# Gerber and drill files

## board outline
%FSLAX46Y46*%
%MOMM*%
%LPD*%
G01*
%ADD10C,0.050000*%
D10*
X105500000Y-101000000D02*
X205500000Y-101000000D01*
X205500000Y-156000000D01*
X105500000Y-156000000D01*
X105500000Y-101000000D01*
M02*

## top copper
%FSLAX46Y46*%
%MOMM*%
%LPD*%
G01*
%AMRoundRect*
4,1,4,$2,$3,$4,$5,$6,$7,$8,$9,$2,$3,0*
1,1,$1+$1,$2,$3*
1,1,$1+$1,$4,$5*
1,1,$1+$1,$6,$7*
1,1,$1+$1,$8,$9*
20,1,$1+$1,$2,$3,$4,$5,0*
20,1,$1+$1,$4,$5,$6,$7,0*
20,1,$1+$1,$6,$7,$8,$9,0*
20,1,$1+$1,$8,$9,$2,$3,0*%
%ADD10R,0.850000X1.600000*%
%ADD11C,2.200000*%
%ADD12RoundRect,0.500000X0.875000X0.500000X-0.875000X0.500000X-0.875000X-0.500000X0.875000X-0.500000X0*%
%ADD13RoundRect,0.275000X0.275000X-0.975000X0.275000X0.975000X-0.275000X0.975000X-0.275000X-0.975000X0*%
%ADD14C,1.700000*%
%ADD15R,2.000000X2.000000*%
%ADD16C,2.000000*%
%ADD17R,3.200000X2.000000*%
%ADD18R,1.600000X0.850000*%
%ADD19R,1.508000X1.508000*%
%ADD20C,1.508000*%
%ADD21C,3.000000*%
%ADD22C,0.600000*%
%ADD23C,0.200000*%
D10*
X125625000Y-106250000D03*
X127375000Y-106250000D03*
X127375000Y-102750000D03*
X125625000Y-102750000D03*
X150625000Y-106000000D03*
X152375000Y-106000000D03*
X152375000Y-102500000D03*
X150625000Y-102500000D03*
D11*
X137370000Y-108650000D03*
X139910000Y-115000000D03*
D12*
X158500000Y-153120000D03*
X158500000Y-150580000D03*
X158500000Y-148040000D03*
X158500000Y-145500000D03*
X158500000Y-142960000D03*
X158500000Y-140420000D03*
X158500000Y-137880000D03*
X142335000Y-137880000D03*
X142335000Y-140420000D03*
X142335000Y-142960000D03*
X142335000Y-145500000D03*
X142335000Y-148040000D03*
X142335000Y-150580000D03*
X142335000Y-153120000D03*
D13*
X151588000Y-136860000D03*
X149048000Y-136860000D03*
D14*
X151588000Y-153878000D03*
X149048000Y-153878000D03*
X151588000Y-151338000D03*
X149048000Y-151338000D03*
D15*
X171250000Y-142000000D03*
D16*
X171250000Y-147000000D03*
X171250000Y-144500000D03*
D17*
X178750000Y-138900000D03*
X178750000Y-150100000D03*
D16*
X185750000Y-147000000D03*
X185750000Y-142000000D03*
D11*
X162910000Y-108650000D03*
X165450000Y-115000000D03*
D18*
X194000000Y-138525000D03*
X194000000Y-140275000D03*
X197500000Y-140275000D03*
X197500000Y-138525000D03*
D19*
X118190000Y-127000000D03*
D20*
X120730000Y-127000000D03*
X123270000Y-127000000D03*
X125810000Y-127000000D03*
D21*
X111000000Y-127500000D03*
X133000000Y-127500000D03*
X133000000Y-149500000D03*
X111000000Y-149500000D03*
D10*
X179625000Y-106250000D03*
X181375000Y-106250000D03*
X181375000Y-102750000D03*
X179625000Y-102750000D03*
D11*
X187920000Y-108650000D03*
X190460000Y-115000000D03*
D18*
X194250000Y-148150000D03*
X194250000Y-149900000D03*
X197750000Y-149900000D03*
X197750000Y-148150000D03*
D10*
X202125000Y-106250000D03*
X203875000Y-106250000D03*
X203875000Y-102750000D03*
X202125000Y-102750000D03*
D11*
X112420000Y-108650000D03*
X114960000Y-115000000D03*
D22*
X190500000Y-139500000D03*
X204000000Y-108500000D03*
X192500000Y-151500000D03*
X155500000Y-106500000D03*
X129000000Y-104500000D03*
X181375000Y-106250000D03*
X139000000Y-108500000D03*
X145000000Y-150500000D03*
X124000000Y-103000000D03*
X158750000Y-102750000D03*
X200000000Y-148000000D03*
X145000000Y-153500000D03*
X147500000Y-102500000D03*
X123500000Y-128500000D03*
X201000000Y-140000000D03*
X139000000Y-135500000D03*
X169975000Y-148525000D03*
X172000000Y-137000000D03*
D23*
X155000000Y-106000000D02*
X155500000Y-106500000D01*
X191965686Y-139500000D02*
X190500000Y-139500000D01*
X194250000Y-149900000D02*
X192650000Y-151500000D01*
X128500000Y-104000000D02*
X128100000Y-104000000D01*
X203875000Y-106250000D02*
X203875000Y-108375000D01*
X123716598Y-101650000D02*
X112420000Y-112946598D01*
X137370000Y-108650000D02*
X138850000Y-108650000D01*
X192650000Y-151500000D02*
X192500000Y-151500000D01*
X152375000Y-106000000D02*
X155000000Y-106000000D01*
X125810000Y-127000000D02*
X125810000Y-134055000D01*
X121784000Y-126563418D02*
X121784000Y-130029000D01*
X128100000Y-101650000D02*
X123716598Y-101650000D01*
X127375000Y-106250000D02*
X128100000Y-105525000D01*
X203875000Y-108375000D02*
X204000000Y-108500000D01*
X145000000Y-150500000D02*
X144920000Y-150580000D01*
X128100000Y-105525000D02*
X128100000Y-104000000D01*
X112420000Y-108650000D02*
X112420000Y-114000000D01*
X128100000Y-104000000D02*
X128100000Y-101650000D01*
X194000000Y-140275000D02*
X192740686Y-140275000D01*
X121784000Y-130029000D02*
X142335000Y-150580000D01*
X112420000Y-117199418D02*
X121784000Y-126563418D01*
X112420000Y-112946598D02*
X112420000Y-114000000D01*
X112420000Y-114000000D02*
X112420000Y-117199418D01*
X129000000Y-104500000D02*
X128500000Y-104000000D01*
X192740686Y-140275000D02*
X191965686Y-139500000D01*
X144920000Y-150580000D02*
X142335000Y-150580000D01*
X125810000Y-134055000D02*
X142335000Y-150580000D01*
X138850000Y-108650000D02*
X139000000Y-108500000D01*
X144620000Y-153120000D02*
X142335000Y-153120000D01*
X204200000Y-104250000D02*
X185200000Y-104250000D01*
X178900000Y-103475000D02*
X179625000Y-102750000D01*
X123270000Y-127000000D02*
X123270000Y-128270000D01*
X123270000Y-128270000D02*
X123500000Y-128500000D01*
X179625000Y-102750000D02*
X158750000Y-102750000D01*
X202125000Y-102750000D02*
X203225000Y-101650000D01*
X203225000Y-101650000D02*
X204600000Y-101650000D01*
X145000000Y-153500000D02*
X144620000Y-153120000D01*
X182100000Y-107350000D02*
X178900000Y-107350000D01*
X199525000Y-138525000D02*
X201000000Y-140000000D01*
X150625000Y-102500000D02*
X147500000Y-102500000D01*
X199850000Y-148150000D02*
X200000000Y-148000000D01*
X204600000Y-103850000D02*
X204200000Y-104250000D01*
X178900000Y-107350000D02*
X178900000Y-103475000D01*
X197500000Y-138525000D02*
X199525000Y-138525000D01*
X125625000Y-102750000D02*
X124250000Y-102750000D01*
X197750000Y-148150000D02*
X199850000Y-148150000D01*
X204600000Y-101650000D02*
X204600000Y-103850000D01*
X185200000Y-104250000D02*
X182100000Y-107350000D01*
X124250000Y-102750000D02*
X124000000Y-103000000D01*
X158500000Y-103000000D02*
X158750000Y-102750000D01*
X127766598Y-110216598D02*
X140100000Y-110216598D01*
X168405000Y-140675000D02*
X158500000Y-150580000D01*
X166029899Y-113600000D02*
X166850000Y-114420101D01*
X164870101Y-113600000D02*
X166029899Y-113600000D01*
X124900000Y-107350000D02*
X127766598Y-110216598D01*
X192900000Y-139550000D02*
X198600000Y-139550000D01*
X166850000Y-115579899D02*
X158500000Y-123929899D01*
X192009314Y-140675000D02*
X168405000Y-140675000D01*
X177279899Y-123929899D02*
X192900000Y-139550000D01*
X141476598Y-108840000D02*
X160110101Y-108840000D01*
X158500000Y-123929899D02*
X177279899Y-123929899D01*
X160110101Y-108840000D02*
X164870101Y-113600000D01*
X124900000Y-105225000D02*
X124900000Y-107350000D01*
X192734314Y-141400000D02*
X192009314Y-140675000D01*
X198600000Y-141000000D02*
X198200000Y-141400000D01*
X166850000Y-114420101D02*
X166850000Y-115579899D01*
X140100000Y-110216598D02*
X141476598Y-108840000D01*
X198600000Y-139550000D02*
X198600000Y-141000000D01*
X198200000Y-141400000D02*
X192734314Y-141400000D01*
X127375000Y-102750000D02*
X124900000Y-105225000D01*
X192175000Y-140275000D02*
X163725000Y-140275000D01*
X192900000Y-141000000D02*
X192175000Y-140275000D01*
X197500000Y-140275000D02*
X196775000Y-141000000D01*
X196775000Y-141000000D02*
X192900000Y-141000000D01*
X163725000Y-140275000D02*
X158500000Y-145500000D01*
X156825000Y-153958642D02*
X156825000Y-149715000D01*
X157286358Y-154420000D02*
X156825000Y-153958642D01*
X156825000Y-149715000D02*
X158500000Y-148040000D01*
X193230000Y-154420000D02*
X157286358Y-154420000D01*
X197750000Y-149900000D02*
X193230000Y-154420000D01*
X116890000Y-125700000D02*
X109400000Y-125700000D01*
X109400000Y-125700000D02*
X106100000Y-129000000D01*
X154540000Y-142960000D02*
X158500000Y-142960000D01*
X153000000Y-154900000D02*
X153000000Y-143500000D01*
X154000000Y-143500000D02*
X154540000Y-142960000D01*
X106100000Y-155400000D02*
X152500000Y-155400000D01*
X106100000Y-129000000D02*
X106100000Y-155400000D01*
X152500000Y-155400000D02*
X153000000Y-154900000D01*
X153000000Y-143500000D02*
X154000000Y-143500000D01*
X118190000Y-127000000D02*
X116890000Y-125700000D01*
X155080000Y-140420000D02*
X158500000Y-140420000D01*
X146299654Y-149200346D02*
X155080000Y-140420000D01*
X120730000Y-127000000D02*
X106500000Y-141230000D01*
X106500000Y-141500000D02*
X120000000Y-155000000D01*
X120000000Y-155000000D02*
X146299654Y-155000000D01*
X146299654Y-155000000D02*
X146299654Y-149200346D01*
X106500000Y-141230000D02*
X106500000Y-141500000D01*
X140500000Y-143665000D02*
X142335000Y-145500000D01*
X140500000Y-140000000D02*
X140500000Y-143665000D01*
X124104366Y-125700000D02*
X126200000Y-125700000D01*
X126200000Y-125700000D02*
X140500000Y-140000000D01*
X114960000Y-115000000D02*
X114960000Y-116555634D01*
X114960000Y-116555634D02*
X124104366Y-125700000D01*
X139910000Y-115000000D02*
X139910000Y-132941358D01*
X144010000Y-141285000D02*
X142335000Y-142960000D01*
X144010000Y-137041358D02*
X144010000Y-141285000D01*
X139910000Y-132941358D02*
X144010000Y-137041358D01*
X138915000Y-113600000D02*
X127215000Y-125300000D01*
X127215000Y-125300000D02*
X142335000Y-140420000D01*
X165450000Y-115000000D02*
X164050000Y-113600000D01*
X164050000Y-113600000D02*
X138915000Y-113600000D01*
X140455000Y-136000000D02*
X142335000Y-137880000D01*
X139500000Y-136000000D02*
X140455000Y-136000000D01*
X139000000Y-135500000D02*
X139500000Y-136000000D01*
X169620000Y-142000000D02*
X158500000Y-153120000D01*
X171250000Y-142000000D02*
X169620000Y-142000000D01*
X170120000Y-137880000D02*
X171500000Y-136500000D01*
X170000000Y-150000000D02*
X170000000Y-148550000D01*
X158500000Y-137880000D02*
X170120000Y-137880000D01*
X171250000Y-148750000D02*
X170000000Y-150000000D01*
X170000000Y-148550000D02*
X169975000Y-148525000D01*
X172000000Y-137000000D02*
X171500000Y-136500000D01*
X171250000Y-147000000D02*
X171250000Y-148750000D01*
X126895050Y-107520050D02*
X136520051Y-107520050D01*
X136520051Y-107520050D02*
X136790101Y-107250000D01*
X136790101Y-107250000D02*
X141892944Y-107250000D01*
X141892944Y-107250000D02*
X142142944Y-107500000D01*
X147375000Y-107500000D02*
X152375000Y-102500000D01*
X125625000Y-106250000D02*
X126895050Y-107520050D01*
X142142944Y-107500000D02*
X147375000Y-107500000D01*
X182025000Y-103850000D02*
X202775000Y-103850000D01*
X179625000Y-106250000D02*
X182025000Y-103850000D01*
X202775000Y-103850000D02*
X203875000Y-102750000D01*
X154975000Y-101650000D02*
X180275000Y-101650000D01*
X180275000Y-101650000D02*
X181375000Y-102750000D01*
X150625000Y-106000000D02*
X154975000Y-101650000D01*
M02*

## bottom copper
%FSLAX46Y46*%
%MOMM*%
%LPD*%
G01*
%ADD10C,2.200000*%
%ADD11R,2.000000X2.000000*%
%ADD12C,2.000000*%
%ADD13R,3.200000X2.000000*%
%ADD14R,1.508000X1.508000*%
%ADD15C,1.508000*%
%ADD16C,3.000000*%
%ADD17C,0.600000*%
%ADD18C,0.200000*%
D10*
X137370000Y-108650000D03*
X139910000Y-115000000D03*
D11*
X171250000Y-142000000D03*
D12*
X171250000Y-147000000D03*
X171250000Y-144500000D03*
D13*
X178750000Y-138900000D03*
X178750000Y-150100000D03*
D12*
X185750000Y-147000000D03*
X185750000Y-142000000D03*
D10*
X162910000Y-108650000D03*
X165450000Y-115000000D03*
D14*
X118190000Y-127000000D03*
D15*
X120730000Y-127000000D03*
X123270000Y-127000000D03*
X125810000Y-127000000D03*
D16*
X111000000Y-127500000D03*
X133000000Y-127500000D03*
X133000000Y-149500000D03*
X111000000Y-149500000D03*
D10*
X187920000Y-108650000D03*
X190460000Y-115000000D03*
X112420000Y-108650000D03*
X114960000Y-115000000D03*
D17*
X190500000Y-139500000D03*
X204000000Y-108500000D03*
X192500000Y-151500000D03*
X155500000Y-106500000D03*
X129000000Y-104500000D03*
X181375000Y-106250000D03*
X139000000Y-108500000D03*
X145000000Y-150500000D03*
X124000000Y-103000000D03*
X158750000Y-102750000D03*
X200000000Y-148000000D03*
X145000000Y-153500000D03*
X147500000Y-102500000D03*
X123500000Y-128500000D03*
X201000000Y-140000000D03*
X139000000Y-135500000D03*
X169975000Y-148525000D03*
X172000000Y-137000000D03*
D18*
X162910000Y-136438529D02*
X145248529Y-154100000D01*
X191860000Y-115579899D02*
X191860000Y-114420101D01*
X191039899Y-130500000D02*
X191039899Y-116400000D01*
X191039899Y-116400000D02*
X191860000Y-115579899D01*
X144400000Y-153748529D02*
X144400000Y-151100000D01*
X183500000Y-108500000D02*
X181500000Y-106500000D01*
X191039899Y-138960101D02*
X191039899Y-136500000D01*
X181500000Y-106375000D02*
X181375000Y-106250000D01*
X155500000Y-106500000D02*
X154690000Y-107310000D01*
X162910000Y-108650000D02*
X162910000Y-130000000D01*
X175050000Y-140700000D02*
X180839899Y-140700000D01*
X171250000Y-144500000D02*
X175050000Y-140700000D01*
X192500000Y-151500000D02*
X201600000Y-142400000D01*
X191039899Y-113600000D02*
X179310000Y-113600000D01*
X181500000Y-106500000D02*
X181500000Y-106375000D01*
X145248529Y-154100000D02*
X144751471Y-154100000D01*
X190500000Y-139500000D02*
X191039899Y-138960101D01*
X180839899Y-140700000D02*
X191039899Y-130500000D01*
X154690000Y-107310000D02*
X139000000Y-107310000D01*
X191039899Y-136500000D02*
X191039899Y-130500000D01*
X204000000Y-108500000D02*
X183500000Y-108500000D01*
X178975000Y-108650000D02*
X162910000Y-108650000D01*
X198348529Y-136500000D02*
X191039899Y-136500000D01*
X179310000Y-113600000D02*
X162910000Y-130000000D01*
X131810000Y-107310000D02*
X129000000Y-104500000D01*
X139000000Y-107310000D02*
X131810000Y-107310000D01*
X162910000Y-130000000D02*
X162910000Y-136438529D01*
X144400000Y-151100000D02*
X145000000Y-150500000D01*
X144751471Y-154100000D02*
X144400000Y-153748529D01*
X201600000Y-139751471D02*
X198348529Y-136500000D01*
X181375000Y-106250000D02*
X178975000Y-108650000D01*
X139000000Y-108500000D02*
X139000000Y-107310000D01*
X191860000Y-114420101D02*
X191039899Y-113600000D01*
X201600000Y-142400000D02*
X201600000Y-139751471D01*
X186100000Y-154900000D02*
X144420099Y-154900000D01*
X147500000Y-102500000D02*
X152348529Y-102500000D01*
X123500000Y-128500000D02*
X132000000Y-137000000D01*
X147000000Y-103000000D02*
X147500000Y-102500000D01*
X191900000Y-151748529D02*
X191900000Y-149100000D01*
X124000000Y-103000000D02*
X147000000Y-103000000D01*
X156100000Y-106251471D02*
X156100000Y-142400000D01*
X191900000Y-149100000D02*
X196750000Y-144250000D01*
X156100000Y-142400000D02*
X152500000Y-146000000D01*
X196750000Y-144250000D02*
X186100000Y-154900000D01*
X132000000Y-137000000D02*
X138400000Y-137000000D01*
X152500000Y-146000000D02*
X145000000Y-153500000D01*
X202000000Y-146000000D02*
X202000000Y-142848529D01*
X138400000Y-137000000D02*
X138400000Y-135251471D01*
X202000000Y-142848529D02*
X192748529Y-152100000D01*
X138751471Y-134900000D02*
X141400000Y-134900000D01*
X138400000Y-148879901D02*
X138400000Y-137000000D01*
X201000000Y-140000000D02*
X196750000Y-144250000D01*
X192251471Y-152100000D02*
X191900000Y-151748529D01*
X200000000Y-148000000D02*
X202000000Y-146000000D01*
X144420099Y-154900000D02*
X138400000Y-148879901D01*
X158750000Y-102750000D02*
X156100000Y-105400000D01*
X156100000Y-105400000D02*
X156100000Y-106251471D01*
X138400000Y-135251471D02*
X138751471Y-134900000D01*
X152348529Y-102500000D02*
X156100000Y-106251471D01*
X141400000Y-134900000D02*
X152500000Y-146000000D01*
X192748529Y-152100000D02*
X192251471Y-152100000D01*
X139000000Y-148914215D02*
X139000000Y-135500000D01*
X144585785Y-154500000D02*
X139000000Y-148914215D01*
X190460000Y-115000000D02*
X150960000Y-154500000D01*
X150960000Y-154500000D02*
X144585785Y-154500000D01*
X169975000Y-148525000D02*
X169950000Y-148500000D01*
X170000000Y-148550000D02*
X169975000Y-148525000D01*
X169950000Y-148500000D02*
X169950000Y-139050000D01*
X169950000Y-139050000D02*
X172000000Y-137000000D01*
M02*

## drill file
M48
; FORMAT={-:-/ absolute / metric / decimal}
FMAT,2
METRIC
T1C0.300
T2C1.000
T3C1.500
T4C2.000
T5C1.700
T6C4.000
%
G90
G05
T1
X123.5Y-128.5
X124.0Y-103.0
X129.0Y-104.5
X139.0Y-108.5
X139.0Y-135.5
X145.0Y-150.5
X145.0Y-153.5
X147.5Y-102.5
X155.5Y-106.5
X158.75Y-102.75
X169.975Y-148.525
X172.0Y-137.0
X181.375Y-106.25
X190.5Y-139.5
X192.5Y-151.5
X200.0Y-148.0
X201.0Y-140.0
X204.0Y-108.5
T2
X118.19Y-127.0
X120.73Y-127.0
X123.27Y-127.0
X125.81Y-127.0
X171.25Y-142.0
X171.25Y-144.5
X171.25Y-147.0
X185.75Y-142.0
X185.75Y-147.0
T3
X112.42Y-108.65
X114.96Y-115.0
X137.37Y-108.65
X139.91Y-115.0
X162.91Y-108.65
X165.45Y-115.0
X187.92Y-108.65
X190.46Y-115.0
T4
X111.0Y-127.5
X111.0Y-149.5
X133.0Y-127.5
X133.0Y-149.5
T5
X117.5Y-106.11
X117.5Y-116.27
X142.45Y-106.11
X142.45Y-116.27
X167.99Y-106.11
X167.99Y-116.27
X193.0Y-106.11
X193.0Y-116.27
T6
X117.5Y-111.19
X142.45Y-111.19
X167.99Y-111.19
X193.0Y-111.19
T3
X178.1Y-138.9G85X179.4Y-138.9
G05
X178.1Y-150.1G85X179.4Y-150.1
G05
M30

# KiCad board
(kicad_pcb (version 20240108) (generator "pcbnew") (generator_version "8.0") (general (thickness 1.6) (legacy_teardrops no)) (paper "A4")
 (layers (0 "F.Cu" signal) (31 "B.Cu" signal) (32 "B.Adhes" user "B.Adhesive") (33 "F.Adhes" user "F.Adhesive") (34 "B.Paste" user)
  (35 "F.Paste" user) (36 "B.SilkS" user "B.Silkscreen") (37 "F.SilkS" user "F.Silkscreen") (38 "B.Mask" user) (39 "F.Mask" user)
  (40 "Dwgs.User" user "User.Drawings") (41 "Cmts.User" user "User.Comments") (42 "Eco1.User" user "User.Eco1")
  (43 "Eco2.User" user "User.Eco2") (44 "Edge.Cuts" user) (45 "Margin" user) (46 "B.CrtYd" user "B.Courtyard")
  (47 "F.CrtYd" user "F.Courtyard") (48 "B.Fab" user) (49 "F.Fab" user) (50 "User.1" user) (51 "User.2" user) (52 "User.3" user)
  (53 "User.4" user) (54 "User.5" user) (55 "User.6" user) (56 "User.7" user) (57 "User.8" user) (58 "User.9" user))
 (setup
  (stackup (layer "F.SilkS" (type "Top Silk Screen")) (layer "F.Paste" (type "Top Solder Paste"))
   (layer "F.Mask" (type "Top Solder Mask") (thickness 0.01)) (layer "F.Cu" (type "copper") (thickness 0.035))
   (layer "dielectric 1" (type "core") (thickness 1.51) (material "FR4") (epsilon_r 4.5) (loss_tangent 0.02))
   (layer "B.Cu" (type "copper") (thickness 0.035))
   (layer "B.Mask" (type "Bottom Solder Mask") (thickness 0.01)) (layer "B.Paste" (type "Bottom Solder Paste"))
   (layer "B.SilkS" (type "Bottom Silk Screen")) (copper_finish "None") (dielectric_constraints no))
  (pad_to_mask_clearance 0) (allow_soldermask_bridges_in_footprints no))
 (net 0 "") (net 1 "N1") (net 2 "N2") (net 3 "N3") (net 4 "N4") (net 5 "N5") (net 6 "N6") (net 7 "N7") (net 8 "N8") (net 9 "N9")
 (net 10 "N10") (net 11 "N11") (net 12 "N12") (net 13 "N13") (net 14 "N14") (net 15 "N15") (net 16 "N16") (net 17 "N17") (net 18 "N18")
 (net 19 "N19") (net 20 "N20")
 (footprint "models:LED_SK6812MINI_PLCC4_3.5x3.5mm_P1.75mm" (layer "F.Cu") (at 126.5 104.5 90)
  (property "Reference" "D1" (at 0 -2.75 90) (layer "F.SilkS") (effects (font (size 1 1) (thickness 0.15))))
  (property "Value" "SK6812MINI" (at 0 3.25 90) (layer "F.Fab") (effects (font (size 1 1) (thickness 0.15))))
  (pad "1" smd rect (at -1.75 -0.875 90) (size 1.6 0.85) (layers "F.Cu" "F.Paste" "F.Mask") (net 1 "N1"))
  (pad "2" smd rect (at -1.75 0.875 90) (size 1.6 0.85) (layers "F.Cu" "F.Paste" "F.Mask") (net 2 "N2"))
  (pad "3" smd rect (at 1.75 0.875 90) (size 1.6 0.85) (layers "F.Cu" "F.Paste" "F.Mask") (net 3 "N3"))
  (pad "4" smd rect (at 1.75 -0.875 90) (size 1.6 0.85) (layers "F.Cu" "F.Paste" "F.Mask") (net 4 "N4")))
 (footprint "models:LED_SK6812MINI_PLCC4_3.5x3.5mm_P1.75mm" (layer "F.Cu") (at 151.5 104.25 90)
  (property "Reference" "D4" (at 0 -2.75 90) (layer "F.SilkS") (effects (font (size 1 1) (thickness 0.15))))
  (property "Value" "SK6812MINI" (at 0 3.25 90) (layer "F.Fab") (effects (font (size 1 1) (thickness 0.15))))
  (pad "1" smd rect (at -1.75 -0.875 90) (size 1.6 0.85) (layers "F.Cu" "F.Paste" "F.Mask") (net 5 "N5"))
  (pad "2" smd rect (at -1.75 0.875 90) (size 1.6 0.85) (layers "F.Cu" "F.Paste" "F.Mask") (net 2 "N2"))
  (pad "3" smd rect (at 1.75 0.875 90) (size 1.6 0.85) (layers "F.Cu" "F.Paste" "F.Mask") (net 1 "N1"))
  (pad "4" smd rect (at 1.75 -0.875 90) (size 1.6 0.85) (layers "F.Cu" "F.Paste" "F.Mask") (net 4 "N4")))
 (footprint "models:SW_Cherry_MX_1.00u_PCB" (layer "F.Cu") (at 137.37 108.65 90)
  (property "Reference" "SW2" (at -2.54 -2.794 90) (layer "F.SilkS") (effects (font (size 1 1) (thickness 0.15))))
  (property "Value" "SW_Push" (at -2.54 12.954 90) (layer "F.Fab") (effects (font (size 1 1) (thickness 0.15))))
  (pad "" np_thru_hole circle (at -7.62 5.08 90) (size 1.7 1.7) (drill 1.7) (layers "*.Cu" "*.Mask"))
  (pad "" np_thru_hole circle (at -2.54 5.08 90) (size 4 4) (drill 4) (layers "*.Cu" "*.Mask"))
  (pad "" np_thru_hole circle (at 2.54 5.08 90) (size 1.7 1.7) (drill 1.7) (layers "*.Cu" "*.Mask"))
  (pad "1" thru_hole circle (at 0 0 90) (size 2.2 2.2) (drill 1.5) (layers "*.Cu" "*.Mask") (remove_unused_layers no) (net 2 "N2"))
  (pad "2" thru_hole circle (at -6.35 2.54 90) (size 2.2 2.2) (drill 1.5) (layers "*.Cu" "*.Mask") (remove_unused_layers no) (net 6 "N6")))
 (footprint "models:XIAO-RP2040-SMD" (layer "F.Cu") (at 150.5 145.5 180)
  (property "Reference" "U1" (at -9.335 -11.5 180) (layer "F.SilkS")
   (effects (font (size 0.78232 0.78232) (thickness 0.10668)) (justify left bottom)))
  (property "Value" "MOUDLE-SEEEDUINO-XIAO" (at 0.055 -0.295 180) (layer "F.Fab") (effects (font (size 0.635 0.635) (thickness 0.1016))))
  (pad "1" smd roundrect (at -8 -7.62 180) (size 2.75 2) (layers "F.Cu" "F.Paste" "F.Mask") (roundrect_rratio 0.25) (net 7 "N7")
   (solder_mask_margin 0.0508) (thermal_bridge_angle 45))
  (pad "2" smd roundrect (at -8 -5.08 180) (size 2.75 2) (layers "F.Cu" "F.Paste" "F.Mask") (roundrect_rratio 0.25) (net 3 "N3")
   (solder_mask_margin 0.0508) (thermal_bridge_angle 45))
  (pad "3" smd roundrect (at -8 -2.54 180) (size 2.75 2) (layers "F.Cu" "F.Paste" "F.Mask") (roundrect_rratio 0.25) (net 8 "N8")
   (solder_mask_margin 0.0508) (thermal_bridge_angle 45))
  (pad "4" smd roundrect (at -8 0 180) (size 2.75 2) (layers "F.Cu" "F.Paste" "F.Mask") (roundrect_rratio 0.25) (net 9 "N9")
   (solder_mask_margin 0.0508) (thermal_bridge_angle 45))
  (pad "5" smd roundrect (at -8 2.54 180) (size 2.75 2) (layers "F.Cu" "F.Paste" "F.Mask") (roundrect_rratio 0.25) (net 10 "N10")
   (solder_mask_margin 0.0508) (thermal_bridge_angle 45))
  (pad "6" smd roundrect (at -8 5.08 180) (size 2.75 2) (layers "F.Cu" "F.Paste" "F.Mask") (roundrect_rratio 0.25) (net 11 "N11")
   (solder_mask_margin 0.0508) (thermal_bridge_angle 45))
  (pad "7" smd roundrect (at -8 7.62 180) (size 2.75 2) (layers "F.Cu" "F.Paste" "F.Mask") (roundrect_rratio 0.25) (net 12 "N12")
   (solder_mask_margin 0.0508) (thermal_bridge_angle 45))
  (pad "8" smd roundrect (at 8.165 7.62 180) (size 2.75 2) (layers "F.Cu" "F.Paste" "F.Mask") (roundrect_rratio 0.25) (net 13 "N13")
   (solder_mask_margin 0.0508) (thermal_bridge_angle 45))
  (pad "9" smd roundrect (at 8.165 5.08 180) (size 2.75 2) (layers "F.Cu" "F.Paste" "F.Mask") (roundrect_rratio 0.25) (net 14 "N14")
   (solder_mask_margin 0.0508) (thermal_bridge_angle 45))
  (pad "10" smd roundrect (at 8.165 2.54 180) (size 2.75 2) (layers "F.Cu" "F.Paste" "F.Mask") (roundrect_rratio 0.25) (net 6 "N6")
   (solder_mask_margin 0.0508) (thermal_bridge_angle 45))
  (pad "11" smd roundrect (at 8.165 0 180) (size 2.75 2) (layers "F.Cu" "F.Paste" "F.Mask") (roundrect_rratio 0.25) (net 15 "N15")
   (solder_mask_margin 0.0508) (thermal_bridge_angle 45))
  (pad "12" smd roundrect (at 8.165 -2.54 180) (size 2.75 2) (layers "F.Cu" "F.Paste" "F.Mask") (roundrect_rratio 0.25) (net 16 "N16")
   (solder_mask_margin 0.0508) (thermal_bridge_angle 45))
  (pad "13" smd roundrect (at 8.165 -5.08 180) (size 2.75 2) (layers "F.Cu" "F.Paste" "F.Mask") (roundrect_rratio 0.25) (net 2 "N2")
   (solder_mask_margin 0.0508) (thermal_bridge_angle 45))
  (pad "14" smd roundrect (at 8.165 -7.62 180) (size 2.75 2) (layers "F.Cu" "F.Paste" "F.Mask") (roundrect_rratio 0.25) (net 4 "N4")
   (solder_mask_margin 0.0508) (thermal_bridge_angle 45))
  (pad "15" smd roundrect (at -1.088 8.64 90) (size 2.5 1.1) (layers "F.Cu" "F.Paste" "F.Mask") (roundrect_rratio 0.25)
   (thermal_bridge_angle 45))
  (pad "16" smd roundrect (at 1.452 8.64 90) (size 2.5 1.1) (layers "F.Cu" "F.Paste" "F.Mask") (roundrect_rratio 0.25)
   (thermal_bridge_angle 45))
  (pad "17" smd circle (at -1.088 -8.378 180) (size 1.7 1.7) (layers "F.Cu" "F.Paste" "F.Mask"))
  (pad "18" smd circle (at 1.452 -8.378 180) (size 1.7 1.7) (layers "F.Cu" "F.Paste" "F.Mask"))
  (pad "19" smd circle (at -1.088 -5.838 180) (size 1.7 1.7) (layers "F.Cu" "F.Paste" "F.Mask"))
  (pad "20" smd circle (at 1.452 -5.838 180) (size 1.7 1.7) (layers "F.Cu" "F.Paste" "F.Mask")))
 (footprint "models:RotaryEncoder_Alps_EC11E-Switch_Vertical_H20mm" (layer "F.Cu") (at 171.25 142)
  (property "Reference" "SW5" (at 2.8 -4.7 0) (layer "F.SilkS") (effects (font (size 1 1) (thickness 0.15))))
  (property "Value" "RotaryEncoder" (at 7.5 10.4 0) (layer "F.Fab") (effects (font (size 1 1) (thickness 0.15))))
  (pad "A" thru_hole rect (at 0 0) (size 2 2) (drill 1) (layers "*.Cu" "*.Mask") (remove_unused_layers no) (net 7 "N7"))
  (pad "B" thru_hole circle (at 0 5) (size 2 2) (drill 1) (layers "*.Cu" "*.Mask") (remove_unused_layers no) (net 12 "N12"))
  (pad "C" thru_hole circle (at 0 2.5) (size 2 2) (drill 1) (layers "*.Cu" "*.Mask") (remove_unused_layers no) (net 2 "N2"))
  (pad "MP" thru_hole rect (at 7.5 -3.1) (size 3.2 2) (drill oval 2.8 1.5) (layers "*.Cu" "*.Mask") (remove_unused_layers no))
  (pad "MP" thru_hole rect (at 7.5 8.1) (size 3.2 2) (drill oval 2.8 1.5) (layers "*.Cu" "*.Mask") (remove_unused_layers no))
  (pad "S1" thru_hole circle (at 14.5 5) (size 2 2) (drill 1) (layers "*.Cu" "*.Mask") (remove_unused_layers no))
  (pad "S2" thru_hole circle (at 14.5 0) (size 2 2) (drill 1) (layers "*.Cu" "*.Mask") (remove_unused_layers no)))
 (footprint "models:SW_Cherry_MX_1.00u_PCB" (layer "F.Cu") (at 162.91 108.65 90)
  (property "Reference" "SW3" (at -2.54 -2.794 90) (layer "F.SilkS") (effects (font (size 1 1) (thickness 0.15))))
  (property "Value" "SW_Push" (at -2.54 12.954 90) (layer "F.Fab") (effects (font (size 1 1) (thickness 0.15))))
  (pad "" np_thru_hole circle (at -7.62 5.08 90) (size 1.7 1.7) (drill 1.7) (layers "*.Cu" "*.Mask"))
  (pad "" np_thru_hole circle (at -2.54 5.08 90) (size 4 4) (drill 4) (layers "*.Cu" "*.Mask"))
  (pad "" np_thru_hole circle (at 2.54 5.08 90) (size 1.7 1.7) (drill 1.7) (layers "*.Cu" "*.Mask"))
  (pad "1" thru_hole circle (at 0 0 90) (size 2.2 2.2) (drill 1.5) (layers "*.Cu" "*.Mask") (remove_unused_layers no) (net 2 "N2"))
  (pad "2" thru_hole circle (at -6.35 2.54 90) (size 2.2 2.2) (drill 1.5) (layers "*.Cu" "*.Mask") (remove_unused_layers no) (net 14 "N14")))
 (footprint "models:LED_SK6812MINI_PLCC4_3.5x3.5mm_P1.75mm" (layer "F.Cu") (at 195.75 139.4)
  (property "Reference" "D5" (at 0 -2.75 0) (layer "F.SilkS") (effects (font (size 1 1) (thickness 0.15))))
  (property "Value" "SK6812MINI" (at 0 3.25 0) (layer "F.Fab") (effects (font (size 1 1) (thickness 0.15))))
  (pad "1" smd rect (at -1.75 -0.875) (size 1.6 0.85) (layers "F.Cu" "F.Paste" "F.Mask") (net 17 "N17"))
  (pad "2" smd rect (at -1.75 0.875) (size 1.6 0.85) (layers "F.Cu" "F.Paste" "F.Mask") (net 2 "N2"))
  (pad "3" smd rect (at 1.75 0.875) (size 1.6 0.85) (layers "F.Cu" "F.Paste" "F.Mask") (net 9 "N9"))
  (pad "4" smd rect (at 1.75 -0.875) (size 1.6 0.85) (layers "F.Cu" "F.Paste" "F.Mask") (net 4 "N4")))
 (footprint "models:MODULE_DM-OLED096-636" (layer "F.Cu") (at 122 138.5)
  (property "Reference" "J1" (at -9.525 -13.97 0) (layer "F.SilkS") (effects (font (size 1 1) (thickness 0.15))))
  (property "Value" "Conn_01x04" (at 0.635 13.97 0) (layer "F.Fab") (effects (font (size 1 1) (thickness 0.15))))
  (pad "1" thru_hole rect (at -3.81 -11.5) (size 1.508 1.508) (drill 1) (layers "*.Cu" "*.Mask") (remove_unused_layers no) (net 10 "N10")
   (solder_mask_margin 0.102))
  (pad "2" thru_hole circle (at -1.27 -11.5) (size 1.508 1.508) (drill 1) (layers "*.Cu" "*.Mask") (remove_unused_layers no) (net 11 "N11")
   (solder_mask_margin 0.102))
  (pad "3" thru_hole circle (at 1.27 -11.5) (size 1.508 1.508) (drill 1) (layers "*.Cu" "*.Mask") (remove_unused_layers no) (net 4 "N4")
   (solder_mask_margin 0.102))
  (pad "4" thru_hole circle (at 3.81 -11.5) (size 1.508 1.508) (drill 1) (layers "*.Cu" "*.Mask") (remove_unused_layers no) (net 2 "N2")
   (solder_mask_margin 0.102))
  (pad "S1" thru_hole circle (at -11 -11) (size 3 3) (drill 2) (layers "*.Cu" "*.Mask") (remove_unused_layers no) (solder_mask_margin 0.102))
  (pad "S2" thru_hole circle (at 11 -11) (size 3 3) (drill 2) (layers "*.Cu" "*.Mask") (remove_unused_layers no) (solder_mask_margin 0.102))
  (pad "S3" thru_hole circle (at 11 11) (size 3 3) (drill 2) (layers "*.Cu" "*.Mask") (remove_unused_layers no) (solder_mask_margin 0.102))
  (pad "S4" thru_hole circle (at -11 11) (size 3 3) (drill 2) (layers "*.Cu" "*.Mask") (remove_unused_layers no) (solder_mask_margin 0.102)))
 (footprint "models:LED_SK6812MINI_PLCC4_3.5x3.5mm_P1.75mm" (layer "F.Cu") (at 180.5 104.5 90)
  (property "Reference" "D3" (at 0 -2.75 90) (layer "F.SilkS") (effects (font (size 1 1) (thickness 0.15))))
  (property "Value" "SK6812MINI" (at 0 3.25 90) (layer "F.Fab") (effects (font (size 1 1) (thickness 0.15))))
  (pad "1" smd rect (at -1.75 -0.875 90) (size 1.6 0.85) (layers "F.Cu" "F.Paste" "F.Mask") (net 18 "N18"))
  (pad "2" smd rect (at -1.75 0.875 90) (size 1.6 0.85) (layers "F.Cu" "F.Paste" "F.Mask") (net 2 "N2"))
  (pad "3" smd rect (at 1.75 0.875 90) (size 1.6 0.85) (layers "F.Cu" "F.Paste" "F.Mask") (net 5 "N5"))
  (pad "4" smd rect (at 1.75 -0.875 90) (size 1.6 0.85) (layers "F.Cu" "F.Paste" "F.Mask") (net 4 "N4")))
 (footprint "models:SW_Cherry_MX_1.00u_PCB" (layer "F.Cu") (at 187.92 108.65 90)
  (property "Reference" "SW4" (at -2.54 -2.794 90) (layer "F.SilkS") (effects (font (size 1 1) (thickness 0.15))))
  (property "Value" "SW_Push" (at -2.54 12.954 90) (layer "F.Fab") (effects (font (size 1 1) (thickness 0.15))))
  (pad "" np_thru_hole circle (at -7.62 5.08 90) (size 1.7 1.7) (drill 1.7) (layers "*.Cu" "*.Mask"))
  (pad "" np_thru_hole circle (at -2.54 5.08 90) (size 4 4) (drill 4) (layers "*.Cu" "*.Mask"))
  (pad "" np_thru_hole circle (at 2.54 5.08 90) (size 1.7 1.7) (drill 1.7) (layers "*.Cu" "*.Mask"))
  (pad "1" thru_hole circle (at 0 0 90) (size 2.2 2.2) (drill 1.5) (layers "*.Cu" "*.Mask") (remove_unused_layers no) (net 2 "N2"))
  (pad "2" thru_hole circle (at -6.35 2.54 90) (size 2.2 2.2) (drill 1.5) (layers "*.Cu" "*.Mask") (remove_unused_layers no) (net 13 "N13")))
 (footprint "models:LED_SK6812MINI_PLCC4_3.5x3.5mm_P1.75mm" (layer "F.Cu") (at 196 149.025)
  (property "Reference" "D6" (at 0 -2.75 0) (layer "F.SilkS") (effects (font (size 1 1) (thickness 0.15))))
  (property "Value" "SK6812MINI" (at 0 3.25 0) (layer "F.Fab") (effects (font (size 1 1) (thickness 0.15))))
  (pad "1" smd rect (at -1.75 -0.875) (size 1.6 0.85) (layers "F.Cu" "F.Paste" "F.Mask") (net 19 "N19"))
  (pad "2" smd rect (at -1.75 0.875) (size 1.6 0.85) (layers "F.Cu" "F.Paste" "F.Mask") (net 2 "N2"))
  (pad "3" smd rect (at 1.75 0.875) (size 1.6 0.85) (layers "F.Cu" "F.Paste" "F.Mask") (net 8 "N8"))
  (pad "4" smd rect (at 1.75 -0.875) (size 1.6 0.85) (layers "F.Cu" "F.Paste" "F.Mask") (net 4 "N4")))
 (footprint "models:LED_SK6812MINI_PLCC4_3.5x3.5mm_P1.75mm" (layer "F.Cu") (at 203 104.5 90)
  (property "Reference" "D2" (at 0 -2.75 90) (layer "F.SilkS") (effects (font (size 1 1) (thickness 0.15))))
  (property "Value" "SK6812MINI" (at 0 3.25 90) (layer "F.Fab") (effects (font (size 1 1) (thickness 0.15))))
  (pad "1" smd rect (at -1.75 -0.875 90) (size 1.6 0.85) (layers "F.Cu" "F.Paste" "F.Mask") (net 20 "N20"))
  (pad "2" smd rect (at -1.75 0.875 90) (size 1.6 0.85) (layers "F.Cu" "F.Paste" "F.Mask") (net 2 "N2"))
  (pad "3" smd rect (at 1.75 0.875 90) (size 1.6 0.85) (layers "F.Cu" "F.Paste" "F.Mask") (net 18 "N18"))
  (pad "4" smd rect (at 1.75 -0.875 90) (size 1.6 0.85) (layers "F.Cu" "F.Paste" "F.Mask") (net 4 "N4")))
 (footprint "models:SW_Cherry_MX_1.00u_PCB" (layer "F.Cu") (at 112.42 108.65 90)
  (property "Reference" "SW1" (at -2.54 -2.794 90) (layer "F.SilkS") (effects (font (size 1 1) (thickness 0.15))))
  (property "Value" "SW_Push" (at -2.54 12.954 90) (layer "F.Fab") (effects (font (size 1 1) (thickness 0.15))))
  (pad "" np_thru_hole circle (at -7.62 5.08 90) (size 1.7 1.7) (drill 1.7) (layers "*.Cu" "*.Mask"))
  (pad "" np_thru_hole circle (at -2.54 5.08 90) (size 4 4) (drill 4) (layers "*.Cu" "*.Mask"))
  (pad "" np_thru_hole circle (at 2.54 5.08 90) (size 1.7 1.7) (drill 1.7) (layers "*.Cu" "*.Mask"))
  (pad "1" thru_hole circle (at 0 0 90) (size 2.2 2.2) (drill 1.5) (layers "*.Cu" "*.Mask") (remove_unused_layers no) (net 2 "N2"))
  (pad "2" thru_hole circle (at -6.35 2.54 90) (size 2.2 2.2) (drill 1.5) (layers "*.Cu" "*.Mask") (remove_unused_layers no) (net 15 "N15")))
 (gr_rect (start 105.5 101) (end 205.5 156) (stroke (width 0.05) (type default)) (fill none) (layer "Edge.Cuts"))
 (segment (start 155 106) (end 155.5 106.5) (width 0.2) (layer "F.Cu") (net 2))
 (segment (start 191.965686 139.5) (end 190.5 139.5) (width 0.2) (layer "F.Cu") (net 2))
 (segment (start 194.25 149.9) (end 192.65 151.5) (width 0.2) (layer "F.Cu") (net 2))
 (segment (start 128.5 104) (end 128.1 104) (width 0.2) (layer "F.Cu") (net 2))
 (segment (start 203.875 106.25) (end 203.875 108.375) (width 0.2) (layer "F.Cu") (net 2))
 (segment (start 123.716598 101.65) (end 112.42 112.946598) (width 0.2) (layer "F.Cu") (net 2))
 (segment (start 137.37 108.65) (end 138.85 108.65) (width 0.2) (layer "F.Cu") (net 2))
 (segment (start 192.65 151.5) (end 192.5 151.5) (width 0.2) (layer "F.Cu") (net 2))
 (segment (start 152.375 106) (end 155 106) (width 0.2) (layer "F.Cu") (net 2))
 (segment (start 125.81 127) (end 125.81 134.055) (width 0.2) (layer "F.Cu") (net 2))
 (segment (start 121.784 126.563418) (end 121.784 130.029) (width 0.2) (layer "F.Cu") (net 2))
 (segment (start 128.1 101.65) (end 123.716598 101.65) (width 0.2) (layer "F.Cu") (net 2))
 (segment (start 127.375 106.25) (end 128.1 105.525) (width 0.2) (layer "F.Cu") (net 2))
 (segment (start 203.875 108.375) (end 204 108.5) (width 0.2) (layer "F.Cu") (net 2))
 (segment (start 145 150.5) (end 144.92 150.58) (width 0.2) (layer "F.Cu") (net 2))
 (segment (start 128.1 105.525) (end 128.1 104) (width 0.2) (layer "F.Cu") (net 2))
 (segment (start 112.42 108.65) (end 112.42 114) (width 0.2) (layer "F.Cu") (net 2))
 (segment (start 128.1 104) (end 128.1 101.65) (width 0.2) (layer "F.Cu") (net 2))
 (segment (start 194 140.275) (end 192.740686 140.275) (width 0.2) (layer "F.Cu") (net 2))
 (segment (start 121.784 130.029) (end 142.335 150.58) (width 0.2) (layer "F.Cu") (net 2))
 (segment (start 112.42 117.199418) (end 121.784 126.563418) (width 0.2) (layer "F.Cu") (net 2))
 (segment (start 112.42 112.946598) (end 112.42 114) (width 0.2) (layer "F.Cu") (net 2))
 (segment (start 112.42 114) (end 112.42 117.199418) (width 0.2) (layer "F.Cu") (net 2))
 (segment (start 129 104.5) (end 128.5 104) (width 0.2) (layer "F.Cu") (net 2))
 (segment (start 192.740686 140.275) (end 191.965686 139.5) (width 0.2) (layer "F.Cu") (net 2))
 (segment (start 144.92 150.58) (end 142.335 150.58) (width 0.2) (layer "F.Cu") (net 2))
 (segment (start 125.81 134.055) (end 142.335 150.58) (width 0.2) (layer "F.Cu") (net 2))
 (segment (start 138.85 108.65) (end 139 108.5) (width 0.2) (layer "F.Cu") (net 2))
 (via (at 190.5 139.5) (size 0.6) (drill 0.3) (layers "F.Cu" "B.Cu") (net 2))
 (via (at 204 108.5) (size 0.6) (drill 0.3) (layers "F.Cu" "B.Cu") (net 2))
 (via (at 192.5 151.5) (size 0.6) (drill 0.3) (layers "F.Cu" "B.Cu") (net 2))
 (via (at 155.5 106.5) (size 0.6) (drill 0.3) (layers "F.Cu" "B.Cu") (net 2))
 (via (at 129 104.5) (size 0.6) (drill 0.3) (layers "F.Cu" "B.Cu") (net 2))
 (via (at 181.375 106.25) (size 0.6) (drill 0.3) (layers "F.Cu" "B.Cu") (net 2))
 (via (at 139 108.5) (size 0.6) (drill 0.3) (layers "F.Cu" "B.Cu") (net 2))
 (via (at 145 150.5) (size 0.6) (drill 0.3) (layers "F.Cu" "B.Cu") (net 2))
 (segment (start 162.91 136.438529) (end 145.248529 154.1) (width 0.2) (layer "B.Cu") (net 2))
 (segment (start 191.86 115.579899) (end 191.86 114.420101) (width 0.2) (layer "B.Cu") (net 2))
 (segment (start 191.039899 130.5) (end 191.039899 116.4) (width 0.2) (layer "B.Cu") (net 2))
 (segment (start 191.039899 116.4) (end 191.86 115.579899) (width 0.2) (layer "B.Cu") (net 2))
 (segment (start 144.4 153.748529) (end 144.4 151.1) (width 0.2) (layer "B.Cu") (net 2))
 (segment (start 183.5 108.5) (end 181.5 106.5) (width 0.2) (layer "B.Cu") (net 2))
 (segment (start 191.039899 138.960101) (end 191.039899 136.5) (width 0.2) (layer "B.Cu") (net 2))
 (segment (start 181.5 106.375) (end 181.375 106.25) (width 0.2) (layer "B.Cu") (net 2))
 (segment (start 155.5 106.5) (end 154.69 107.31) (width 0.2) (layer "B.Cu") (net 2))
 (segment (start 162.91 108.65) (end 162.91 130) (width 0.2) (layer "B.Cu") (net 2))
 (segment (start 175.05 140.7) (end 180.839899 140.7) (width 0.2) (layer "B.Cu") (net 2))
 (segment (start 171.25 144.5) (end 175.05 140.7) (width 0.2) (layer "B.Cu") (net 2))
 (segment (start 192.5 151.5) (end 201.6 142.4) (width 0.2) (layer "B.Cu") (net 2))
 (segment (start 191.039899 113.6) (end 179.31 113.6) (width 0.2) (layer "B.Cu") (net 2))
 (segment (start 181.5 106.5) (end 181.5 106.375) (width 0.2) (layer "B.Cu") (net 2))
 (segment (start 145.248529 154.1) (end 144.751471 154.1) (width 0.2) (layer "B.Cu") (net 2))
 (segment (start 190.5 139.5) (end 191.039899 138.960101) (width 0.2) (layer "B.Cu") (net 2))
 (segment (start 180.839899 140.7) (end 191.039899 130.5) (width 0.2) (layer "B.Cu") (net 2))
 (segment (start 154.69 107.31) (end 139 107.31) (width 0.2) (layer "B.Cu") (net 2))
 (segment (start 191.039899 136.5) (end 191.039899 130.5) (width 0.2) (layer "B.Cu") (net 2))
 (segment (start 204 108.5) (end 183.5 108.5) (width 0.2) (layer "B.Cu") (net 2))
 (segment (start 178.975 108.65) (end 162.91 108.65) (width 0.2) (layer "B.Cu") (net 2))
 (segment (start 198.348529 136.5) (end 191.039899 136.5) (width 0.2) (layer "B.Cu") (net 2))
 (segment (start 179.31 113.6) (end 162.91 130) (width 0.2) (layer "B.Cu") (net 2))
 (segment (start 131.81 107.31) (end 129 104.5) (width 0.2) (layer "B.Cu") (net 2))
 (segment (start 139 107.31) (end 131.81 107.31) (width 0.2) (layer "B.Cu") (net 2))
 (segment (start 162.91 130) (end 162.91 136.438529) (width 0.2) (layer "B.Cu") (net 2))
 (segment (start 144.4 151.1) (end 145 150.5) (width 0.2) (layer "B.Cu") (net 2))
 (segment (start 144.751471 154.1) (end 144.4 153.748529) (width 0.2) (layer "B.Cu") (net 2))
 (segment (start 201.6 139.751471) (end 198.348529 136.5) (width 0.2) (layer "B.Cu") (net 2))
 (segment (start 181.375 106.25) (end 178.975 108.65) (width 0.2) (layer "B.Cu") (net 2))
 (segment (start 139 108.5) (end 139 107.31) (width 0.2) (layer "B.Cu") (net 2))
 (segment (start 191.86 114.420101) (end 191.039899 113.6) (width 0.2) (layer "B.Cu") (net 2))
 (segment (start 201.6 142.4) (end 201.6 139.751471) (width 0.2) (layer "B.Cu") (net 2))
 (segment (start 144.62 153.12) (end 142.335 153.12) (width 0.2) (layer "F.Cu") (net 4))
 (segment (start 204.2 104.25) (end 185.2 104.25) (width 0.2) (layer "F.Cu") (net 4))
 (segment (start 178.9 103.475) (end 179.625 102.75) (width 0.2) (layer "F.Cu") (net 4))
 (segment (start 123.27 127) (end 123.27 128.27) (width 0.2) (layer "F.Cu") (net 4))
 (segment (start 123.27 128.27) (end 123.5 128.5) (width 0.2) (layer "F.Cu") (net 4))
 (segment (start 179.625 102.75) (end 158.75 102.75) (width 0.2) (layer "F.Cu") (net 4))
 (segment (start 202.125 102.75) (end 203.225 101.65) (width 0.2) (layer "F.Cu") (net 4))
 (segment (start 203.225 101.65) (end 204.6 101.65) (width 0.2) (layer "F.Cu") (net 4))
 (segment (start 145 153.5) (end 144.62 153.12) (width 0.2) (layer "F.Cu") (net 4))
 (segment (start 182.1 107.35) (end 178.9 107.35) (width 0.2) (layer "F.Cu") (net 4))
 (segment (start 199.525 138.525) (end 201 140) (width 0.2) (layer "F.Cu") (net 4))
 (segment (start 150.625 102.5) (end 147.5 102.5) (width 0.2) (layer "F.Cu") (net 4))
 (segment (start 199.85 148.15) (end 200 148) (width 0.2) (layer "F.Cu") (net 4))
 (segment (start 204.6 103.85) (end 204.2 104.25) (width 0.2) (layer "F.Cu") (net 4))
 (segment (start 178.9 107.35) (end 178.9 103.475) (width 0.2) (layer "F.Cu") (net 4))
 (segment (start 197.5 138.525) (end 199.525 138.525) (width 0.2) (layer "F.Cu") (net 4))
 (segment (start 125.625 102.75) (end 124.25 102.75) (width 0.2) (layer "F.Cu") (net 4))
 (segment (start 197.75 148.15) (end 199.85 148.15) (width 0.2) (layer "F.Cu") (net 4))
 (segment (start 204.6 101.65) (end 204.6 103.85) (width 0.2) (layer "F.Cu") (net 4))
 (segment (start 185.2 104.25) (end 182.1 107.35) (width 0.2) (layer "F.Cu") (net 4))
 (segment (start 124.25 102.75) (end 124 103) (width 0.2) (layer "F.Cu") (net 4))
 (segment (start 158.5 103) (end 158.75 102.75) (width 0.2) (layer "F.Cu") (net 4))
 (via (at 124 103) (size 0.6) (drill 0.3) (layers "F.Cu" "B.Cu") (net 4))
 (via (at 158.75 102.75) (size 0.6) (drill 0.3) (layers "F.Cu" "B.Cu") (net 4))
 (via (at 200 148) (size 0.6) (drill 0.3) (layers "F.Cu" "B.Cu") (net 4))
 (via (at 145 153.5) (size 0.6) (drill 0.3) (layers "F.Cu" "B.Cu") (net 4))
 (via (at 147.5 102.5) (size 0.6) (drill 0.3) (layers "F.Cu" "B.Cu") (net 4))
 (via (at 123.5 128.5) (size 0.6) (drill 0.3) (layers "F.Cu" "B.Cu") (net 4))
 (via (at 201 140) (size 0.6) (drill 0.3) (layers "F.Cu" "B.Cu") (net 4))
 (segment (start 186.1 154.9) (end 144.420099 154.9) (width 0.2) (layer "B.Cu") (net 4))
 (segment (start 147.5 102.5) (end 152.348529 102.5) (width 0.2) (layer "B.Cu") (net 4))
 (segment (start 123.5 128.5) (end 132 137) (width 0.2) (layer "B.Cu") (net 4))
 (segment (start 147 103) (end 147.5 102.5) (width 0.2) (layer "B.Cu") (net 4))
 (segment (start 191.9 151.748529) (end 191.9 149.1) (width 0.2) (layer "B.Cu") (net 4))
 (segment (start 124 103) (end 147 103) (width 0.2) (layer "B.Cu") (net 4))
 (segment (start 156.1 106.251471) (end 156.1 142.4) (width 0.2) (layer "B.Cu") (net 4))
 (segment (start 191.9 149.1) (end 196.75 144.25) (width 0.2) (layer "B.Cu") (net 4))
 (segment (start 156.1 142.4) (end 152.5 146) (width 0.2) (layer "B.Cu") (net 4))
 (segment (start 196.75 144.25) (end 186.1 154.9) (width 0.2) (layer "B.Cu") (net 4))
 (segment (start 132 137) (end 138.4 137) (width 0.2) (layer "B.Cu") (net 4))
 (segment (start 152.5 146) (end 145 153.5) (width 0.2) (layer "B.Cu") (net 4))
 (segment (start 202 146) (end 202 142.848529) (width 0.2) (layer "B.Cu") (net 4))
 (segment (start 138.4 137) (end 138.4 135.251471) (width 0.2) (layer "B.Cu") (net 4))
 (segment (start 202 142.848529) (end 192.748529 152.1) (width 0.2) (layer "B.Cu") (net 4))
 (segment (start 138.751471 134.9) (end 141.4 134.9) (width 0.2) (layer "B.Cu") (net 4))
 (segment (start 138.4 148.879901) (end 138.4 137) (width 0.2) (layer "B.Cu") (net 4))
 (segment (start 201 140) (end 196.75 144.25) (width 0.2) (layer "B.Cu") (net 4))
 (segment (start 192.251471 152.1) (end 191.9 151.748529) (width 0.2) (layer "B.Cu") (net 4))
 (segment (start 200 148) (end 202 146) (width 0.2) (layer "B.Cu") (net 4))
 (segment (start 144.420099 154.9) (end 138.4 148.879901) (width 0.2) (layer "B.Cu") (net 4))
 (segment (start 158.75 102.75) (end 156.1 105.4) (width 0.2) (layer "B.Cu") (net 4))
 (segment (start 156.1 105.4) (end 156.1 106.251471) (width 0.2) (layer "B.Cu") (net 4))
 (segment (start 138.4 135.251471) (end 138.751471 134.9) (width 0.2) (layer "B.Cu") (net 4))
 (segment (start 152.348529 102.5) (end 156.1 106.251471) (width 0.2) (layer "B.Cu") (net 4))
 (segment (start 141.4 134.9) (end 152.5 146) (width 0.2) (layer "B.Cu") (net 4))
 (segment (start 192.748529 152.1) (end 192.251471 152.1) (width 0.2) (layer "B.Cu") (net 4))
 (segment (start 127.766598 110.216598) (end 140.1 110.216598) (width 0.2) (layer "F.Cu") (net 3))
 (segment (start 168.405 140.675) (end 158.5 150.58) (width 0.2) (layer "F.Cu") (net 3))
 (segment (start 166.029899 113.6) (end 166.85 114.420101) (width 0.2) (layer "F.Cu") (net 3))
 (segment (start 164.870101 113.6) (end 166.029899 113.6) (width 0.2) (layer "F.Cu") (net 3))
 (segment (start 124.9 107.35) (end 127.766598 110.216598) (width 0.2) (layer "F.Cu") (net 3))
 (segment (start 192.9 139.55) (end 198.6 139.55) (width 0.2) (layer "F.Cu") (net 3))
 (segment (start 166.85 115.579899) (end 158.5 123.929899) (width 0.2) (layer "F.Cu") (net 3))
 (segment (start 192.009314 140.675) (end 168.405 140.675) (width 0.2) (layer "F.Cu") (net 3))
 (segment (start 177.279899 123.929899) (end 192.9 139.55) (width 0.2) (layer "F.Cu") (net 3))
 (segment (start 141.476598 108.84) (end 160.110101 108.84) (width 0.2) (layer "F.Cu") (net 3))
 (segment (start 158.5 123.929899) (end 177.279899 123.929899) (width 0.2) (layer "F.Cu") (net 3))
 (segment (start 160.110101 108.84) (end 164.870101 113.6) (width 0.2) (layer "F.Cu") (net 3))
 (segment (start 124.9 105.225) (end 124.9 107.35) (width 0.2) (layer "F.Cu") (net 3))
 (segment (start 192.734314 141.4) (end 192.009314 140.675) (width 0.2) (layer "F.Cu") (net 3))
 (segment (start 198.6 141) (end 198.2 141.4) (width 0.2) (layer "F.Cu") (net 3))
 (segment (start 166.85 114.420101) (end 166.85 115.579899) (width 0.2) (layer "F.Cu") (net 3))
 (segment (start 140.1 110.216598) (end 141.476598 108.84) (width 0.2) (layer "F.Cu") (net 3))
 (segment (start 198.6 139.55) (end 198.6 141) (width 0.2) (layer "F.Cu") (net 3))
 (segment (start 198.2 141.4) (end 192.734314 141.4) (width 0.2) (layer "F.Cu") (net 3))
 (segment (start 127.375 102.75) (end 124.9 105.225) (width 0.2) (layer "F.Cu") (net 3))
 (segment (start 192.175 140.275) (end 163.725 140.275) (width 0.2) (layer "F.Cu") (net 9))
 (segment (start 192.9 141) (end 192.175 140.275) (width 0.2) (layer "F.Cu") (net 9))
 (segment (start 197.5 140.275) (end 196.775 141) (width 0.2) (layer "F.Cu") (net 9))
 (segment (start 196.775 141) (end 192.9 141) (width 0.2) (layer "F.Cu") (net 9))
 (segment (start 163.725 140.275) (end 158.5 145.5) (width 0.2) (layer "F.Cu") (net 9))
 (segment (start 156.825 153.958642) (end 156.825 149.715) (width 0.2) (layer "F.Cu") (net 8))
 (segment (start 157.286358 154.42) (end 156.825 153.958642) (width 0.2) (layer "F.Cu") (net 8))
 (segment (start 156.825 149.715) (end 158.5 148.04) (width 0.2) (layer "F.Cu") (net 8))
 (segment (start 193.23 154.42) (end 157.286358 154.42) (width 0.2) (layer "F.Cu") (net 8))
 (segment (start 197.75 149.9) (end 193.23 154.42) (width 0.2) (layer "F.Cu") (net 8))
 (segment (start 116.89 125.7) (end 109.4 125.7) (width 0.2) (layer "F.Cu") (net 10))
 (segment (start 109.4 125.7) (end 106.1 129) (width 0.2) (layer "F.Cu") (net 10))
 (segment (start 154.54 142.96) (end 158.5 142.96) (width 0.2) (layer "F.Cu") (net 10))
 (segment (start 153 154.9) (end 153 143.5) (width 0.2) (layer "F.Cu") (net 10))
 (segment (start 154 143.5) (end 154.54 142.96) (width 0.2) (layer "F.Cu") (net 10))
 (segment (start 106.1 155.4) (end 152.5 155.4) (width 0.2) (layer "F.Cu") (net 10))
 (segment (start 106.1 129) (end 106.1 155.4) (width 0.2) (layer "F.Cu") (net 10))
 (segment (start 152.5 155.4) (end 153 154.9) (width 0.2) (layer "F.Cu") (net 10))
 (segment (start 153 143.5) (end 154 143.5) (width 0.2) (layer "F.Cu") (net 10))
 (segment (start 118.19 127) (end 116.89 125.7) (width 0.2) (layer "F.Cu") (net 10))
 (segment (start 155.08 140.42) (end 158.5 140.42) (width 0.2) (layer "F.Cu") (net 11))
 (segment (start 146.299654 149.200346) (end 155.08 140.42) (width 0.2) (layer "F.Cu") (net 11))
 (segment (start 120.73 127) (end 106.5 141.23) (width 0.2) (layer "F.Cu") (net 11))
 (segment (start 106.5 141.5) (end 120 155) (width 0.2) (layer "F.Cu") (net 11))
 (segment (start 120 155) (end 146.299654 155) (width 0.2) (layer "F.Cu") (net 11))
 (segment (start 146.299654 155) (end 146.299654 149.200346) (width 0.2) (layer "F.Cu") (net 11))
 (segment (start 106.5 141.23) (end 106.5 141.5) (width 0.2) (layer "F.Cu") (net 11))
 (segment (start 140.5 143.665) (end 142.335 145.5) (width 0.2) (layer "F.Cu") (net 15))
 (segment (start 140.5 140) (end 140.5 143.665) (width 0.2) (layer "F.Cu") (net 15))
 (segment (start 124.104366 125.7) (end 126.2 125.7) (width 0.2) (layer "F.Cu") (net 15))
 (segment (start 126.2 125.7) (end 140.5 140) (width 0.2) (layer "F.Cu") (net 15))
 (segment (start 114.96 115) (end 114.96 116.555634) (width 0.2) (layer "F.Cu") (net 15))
 (segment (start 114.96 116.555634) (end 124.104366 125.7) (width 0.2) (layer "F.Cu") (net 15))
 (segment (start 139.91 115) (end 139.91 132.941358) (width 0.2) (layer "F.Cu") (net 6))
 (segment (start 144.01 141.285) (end 142.335 142.96) (width 0.2) (layer "F.Cu") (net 6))
 (segment (start 144.01 137.041358) (end 144.01 141.285) (width 0.2) (layer "F.Cu") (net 6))
 (segment (start 139.91 132.941358) (end 144.01 137.041358) (width 0.2) (layer "F.Cu") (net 6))
 (segment (start 138.915 113.6) (end 127.215 125.3) (width 0.2) (layer "F.Cu") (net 14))
 (segment (start 127.215 125.3) (end 142.335 140.42) (width 0.2) (layer "F.Cu") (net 14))
 (segment (start 165.45 115) (end 164.05 113.6) (width 0.2) (layer "F.Cu") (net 14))
 (segment (start 164.05 113.6) (end 138.915 113.6) (width 0.2) (layer "F.Cu") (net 14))
 (segment (start 140.455 136) (end 142.335 137.88) (width 0.2) (layer "F.Cu") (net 13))
 (segment (start 139.5 136) (end 140.455 136) (width 0.2) (layer "F.Cu") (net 13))
 (segment (start 139 135.5) (end 139.5 136) (width 0.2) (layer "F.Cu") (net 13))
 (via (at 139 135.5) (size 0.6) (drill 0.3) (layers "F.Cu" "B.Cu") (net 13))
 (segment (start 139 148.914215) (end 139 135.5) (width 0.2) (layer "B.Cu") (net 13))
 (segment (start 144.585785 154.5) (end 139 148.914215) (width 0.2) (layer "B.Cu") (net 13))
 (segment (start 190.46 115) (end 150.96 154.5) (width 0.2) (layer "B.Cu") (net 13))
 (segment (start 150.96 154.5) (end 144.585785 154.5) (width 0.2) (layer "B.Cu") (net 13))
 (segment (start 169.62 142) (end 158.5 153.12) (width 0.2) (layer "F.Cu") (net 7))
 (segment (start 171.25 142) (end 169.62 142) (width 0.2) (layer "F.Cu") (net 7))
 (segment (start 170.12 137.88) (end 171.5 136.5) (width 0.2) (layer "F.Cu") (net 12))
 (segment (start 170 150) (end 170 148.55) (width 0.2) (layer "F.Cu") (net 12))
 (segment (start 158.5 137.88) (end 170.12 137.88) (width 0.2) (layer "F.Cu") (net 12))
 (segment (start 171.25 148.75) (end 170 150) (width 0.2) (layer "F.Cu") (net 12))
 (segment (start 170 148.55) (end 169.975 148.525) (width 0.2) (layer "F.Cu") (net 12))
 (segment (start 172 137) (end 171.5 136.5) (width 0.2) (layer "F.Cu") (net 12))
 (segment (start 171.25 147) (end 171.25 148.75) (width 0.2) (layer "F.Cu") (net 12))
 (via (at 169.975 148.525) (size 0.6) (drill 0.3) (layers "F.Cu" "B.Cu") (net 12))
 (via (at 172 137) (size 0.6) (drill 0.3) (layers "F.Cu" "B.Cu") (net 12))
 (segment (start 169.975 148.525) (end 169.95 148.5) (width 0.2) (layer "B.Cu") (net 12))
 (segment (start 170 148.55) (end 169.975 148.525) (width 0.2) (layer "B.Cu") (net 12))
 (segment (start 169.95 148.5) (end 169.95 139.05) (width 0.2) (layer "B.Cu") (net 12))
 (segment (start 169.95 139.05) (end 172 137) (width 0.2) (layer "B.Cu") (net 12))
 (segment (start 126.89505 107.52005) (end 136.520051 107.52005) (width 0.2) (layer "F.Cu") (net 1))
 (segment (start 136.520051 107.52005) (end 136.790101 107.25) (width 0.2) (layer "F.Cu") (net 1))
 (segment (start 136.790101 107.25) (end 141.892944 107.25) (width 0.2) (layer "F.Cu") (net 1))
 (segment (start 141.892944 107.25) (end 142.142944 107.5) (width 0.2) (layer "F.Cu") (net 1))
 (segment (start 147.375 107.5) (end 152.375 102.5) (width 0.2) (layer "F.Cu") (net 1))
 (segment (start 125.625 106.25) (end 126.89505 107.52005) (width 0.2) (layer "F.Cu") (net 1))
 (segment (start 142.142944 107.5) (end 147.375 107.5) (width 0.2) (layer "F.Cu") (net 1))
 (segment (start 182.025 103.85) (end 202.775 103.85) (width 0.2) (layer "F.Cu") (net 18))
 (segment (start 179.625 106.25) (end 182.025 103.85) (width 0.2) (layer "F.Cu") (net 18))
 (segment (start 202.775 103.85) (end 203.875 102.75) (width 0.2) (layer "F.Cu") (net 18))
 (segment (start 154.975 101.65) (end 180.275 101.65) (width 0.2) (layer "F.Cu") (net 5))
 (segment (start 180.275 101.65) (end 181.375 102.75) (width 0.2) (layer "F.Cu") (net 5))
 (segment (start 150.625 106) (end 154.975 101.65) (width 0.2) (layer "F.Cu") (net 5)))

